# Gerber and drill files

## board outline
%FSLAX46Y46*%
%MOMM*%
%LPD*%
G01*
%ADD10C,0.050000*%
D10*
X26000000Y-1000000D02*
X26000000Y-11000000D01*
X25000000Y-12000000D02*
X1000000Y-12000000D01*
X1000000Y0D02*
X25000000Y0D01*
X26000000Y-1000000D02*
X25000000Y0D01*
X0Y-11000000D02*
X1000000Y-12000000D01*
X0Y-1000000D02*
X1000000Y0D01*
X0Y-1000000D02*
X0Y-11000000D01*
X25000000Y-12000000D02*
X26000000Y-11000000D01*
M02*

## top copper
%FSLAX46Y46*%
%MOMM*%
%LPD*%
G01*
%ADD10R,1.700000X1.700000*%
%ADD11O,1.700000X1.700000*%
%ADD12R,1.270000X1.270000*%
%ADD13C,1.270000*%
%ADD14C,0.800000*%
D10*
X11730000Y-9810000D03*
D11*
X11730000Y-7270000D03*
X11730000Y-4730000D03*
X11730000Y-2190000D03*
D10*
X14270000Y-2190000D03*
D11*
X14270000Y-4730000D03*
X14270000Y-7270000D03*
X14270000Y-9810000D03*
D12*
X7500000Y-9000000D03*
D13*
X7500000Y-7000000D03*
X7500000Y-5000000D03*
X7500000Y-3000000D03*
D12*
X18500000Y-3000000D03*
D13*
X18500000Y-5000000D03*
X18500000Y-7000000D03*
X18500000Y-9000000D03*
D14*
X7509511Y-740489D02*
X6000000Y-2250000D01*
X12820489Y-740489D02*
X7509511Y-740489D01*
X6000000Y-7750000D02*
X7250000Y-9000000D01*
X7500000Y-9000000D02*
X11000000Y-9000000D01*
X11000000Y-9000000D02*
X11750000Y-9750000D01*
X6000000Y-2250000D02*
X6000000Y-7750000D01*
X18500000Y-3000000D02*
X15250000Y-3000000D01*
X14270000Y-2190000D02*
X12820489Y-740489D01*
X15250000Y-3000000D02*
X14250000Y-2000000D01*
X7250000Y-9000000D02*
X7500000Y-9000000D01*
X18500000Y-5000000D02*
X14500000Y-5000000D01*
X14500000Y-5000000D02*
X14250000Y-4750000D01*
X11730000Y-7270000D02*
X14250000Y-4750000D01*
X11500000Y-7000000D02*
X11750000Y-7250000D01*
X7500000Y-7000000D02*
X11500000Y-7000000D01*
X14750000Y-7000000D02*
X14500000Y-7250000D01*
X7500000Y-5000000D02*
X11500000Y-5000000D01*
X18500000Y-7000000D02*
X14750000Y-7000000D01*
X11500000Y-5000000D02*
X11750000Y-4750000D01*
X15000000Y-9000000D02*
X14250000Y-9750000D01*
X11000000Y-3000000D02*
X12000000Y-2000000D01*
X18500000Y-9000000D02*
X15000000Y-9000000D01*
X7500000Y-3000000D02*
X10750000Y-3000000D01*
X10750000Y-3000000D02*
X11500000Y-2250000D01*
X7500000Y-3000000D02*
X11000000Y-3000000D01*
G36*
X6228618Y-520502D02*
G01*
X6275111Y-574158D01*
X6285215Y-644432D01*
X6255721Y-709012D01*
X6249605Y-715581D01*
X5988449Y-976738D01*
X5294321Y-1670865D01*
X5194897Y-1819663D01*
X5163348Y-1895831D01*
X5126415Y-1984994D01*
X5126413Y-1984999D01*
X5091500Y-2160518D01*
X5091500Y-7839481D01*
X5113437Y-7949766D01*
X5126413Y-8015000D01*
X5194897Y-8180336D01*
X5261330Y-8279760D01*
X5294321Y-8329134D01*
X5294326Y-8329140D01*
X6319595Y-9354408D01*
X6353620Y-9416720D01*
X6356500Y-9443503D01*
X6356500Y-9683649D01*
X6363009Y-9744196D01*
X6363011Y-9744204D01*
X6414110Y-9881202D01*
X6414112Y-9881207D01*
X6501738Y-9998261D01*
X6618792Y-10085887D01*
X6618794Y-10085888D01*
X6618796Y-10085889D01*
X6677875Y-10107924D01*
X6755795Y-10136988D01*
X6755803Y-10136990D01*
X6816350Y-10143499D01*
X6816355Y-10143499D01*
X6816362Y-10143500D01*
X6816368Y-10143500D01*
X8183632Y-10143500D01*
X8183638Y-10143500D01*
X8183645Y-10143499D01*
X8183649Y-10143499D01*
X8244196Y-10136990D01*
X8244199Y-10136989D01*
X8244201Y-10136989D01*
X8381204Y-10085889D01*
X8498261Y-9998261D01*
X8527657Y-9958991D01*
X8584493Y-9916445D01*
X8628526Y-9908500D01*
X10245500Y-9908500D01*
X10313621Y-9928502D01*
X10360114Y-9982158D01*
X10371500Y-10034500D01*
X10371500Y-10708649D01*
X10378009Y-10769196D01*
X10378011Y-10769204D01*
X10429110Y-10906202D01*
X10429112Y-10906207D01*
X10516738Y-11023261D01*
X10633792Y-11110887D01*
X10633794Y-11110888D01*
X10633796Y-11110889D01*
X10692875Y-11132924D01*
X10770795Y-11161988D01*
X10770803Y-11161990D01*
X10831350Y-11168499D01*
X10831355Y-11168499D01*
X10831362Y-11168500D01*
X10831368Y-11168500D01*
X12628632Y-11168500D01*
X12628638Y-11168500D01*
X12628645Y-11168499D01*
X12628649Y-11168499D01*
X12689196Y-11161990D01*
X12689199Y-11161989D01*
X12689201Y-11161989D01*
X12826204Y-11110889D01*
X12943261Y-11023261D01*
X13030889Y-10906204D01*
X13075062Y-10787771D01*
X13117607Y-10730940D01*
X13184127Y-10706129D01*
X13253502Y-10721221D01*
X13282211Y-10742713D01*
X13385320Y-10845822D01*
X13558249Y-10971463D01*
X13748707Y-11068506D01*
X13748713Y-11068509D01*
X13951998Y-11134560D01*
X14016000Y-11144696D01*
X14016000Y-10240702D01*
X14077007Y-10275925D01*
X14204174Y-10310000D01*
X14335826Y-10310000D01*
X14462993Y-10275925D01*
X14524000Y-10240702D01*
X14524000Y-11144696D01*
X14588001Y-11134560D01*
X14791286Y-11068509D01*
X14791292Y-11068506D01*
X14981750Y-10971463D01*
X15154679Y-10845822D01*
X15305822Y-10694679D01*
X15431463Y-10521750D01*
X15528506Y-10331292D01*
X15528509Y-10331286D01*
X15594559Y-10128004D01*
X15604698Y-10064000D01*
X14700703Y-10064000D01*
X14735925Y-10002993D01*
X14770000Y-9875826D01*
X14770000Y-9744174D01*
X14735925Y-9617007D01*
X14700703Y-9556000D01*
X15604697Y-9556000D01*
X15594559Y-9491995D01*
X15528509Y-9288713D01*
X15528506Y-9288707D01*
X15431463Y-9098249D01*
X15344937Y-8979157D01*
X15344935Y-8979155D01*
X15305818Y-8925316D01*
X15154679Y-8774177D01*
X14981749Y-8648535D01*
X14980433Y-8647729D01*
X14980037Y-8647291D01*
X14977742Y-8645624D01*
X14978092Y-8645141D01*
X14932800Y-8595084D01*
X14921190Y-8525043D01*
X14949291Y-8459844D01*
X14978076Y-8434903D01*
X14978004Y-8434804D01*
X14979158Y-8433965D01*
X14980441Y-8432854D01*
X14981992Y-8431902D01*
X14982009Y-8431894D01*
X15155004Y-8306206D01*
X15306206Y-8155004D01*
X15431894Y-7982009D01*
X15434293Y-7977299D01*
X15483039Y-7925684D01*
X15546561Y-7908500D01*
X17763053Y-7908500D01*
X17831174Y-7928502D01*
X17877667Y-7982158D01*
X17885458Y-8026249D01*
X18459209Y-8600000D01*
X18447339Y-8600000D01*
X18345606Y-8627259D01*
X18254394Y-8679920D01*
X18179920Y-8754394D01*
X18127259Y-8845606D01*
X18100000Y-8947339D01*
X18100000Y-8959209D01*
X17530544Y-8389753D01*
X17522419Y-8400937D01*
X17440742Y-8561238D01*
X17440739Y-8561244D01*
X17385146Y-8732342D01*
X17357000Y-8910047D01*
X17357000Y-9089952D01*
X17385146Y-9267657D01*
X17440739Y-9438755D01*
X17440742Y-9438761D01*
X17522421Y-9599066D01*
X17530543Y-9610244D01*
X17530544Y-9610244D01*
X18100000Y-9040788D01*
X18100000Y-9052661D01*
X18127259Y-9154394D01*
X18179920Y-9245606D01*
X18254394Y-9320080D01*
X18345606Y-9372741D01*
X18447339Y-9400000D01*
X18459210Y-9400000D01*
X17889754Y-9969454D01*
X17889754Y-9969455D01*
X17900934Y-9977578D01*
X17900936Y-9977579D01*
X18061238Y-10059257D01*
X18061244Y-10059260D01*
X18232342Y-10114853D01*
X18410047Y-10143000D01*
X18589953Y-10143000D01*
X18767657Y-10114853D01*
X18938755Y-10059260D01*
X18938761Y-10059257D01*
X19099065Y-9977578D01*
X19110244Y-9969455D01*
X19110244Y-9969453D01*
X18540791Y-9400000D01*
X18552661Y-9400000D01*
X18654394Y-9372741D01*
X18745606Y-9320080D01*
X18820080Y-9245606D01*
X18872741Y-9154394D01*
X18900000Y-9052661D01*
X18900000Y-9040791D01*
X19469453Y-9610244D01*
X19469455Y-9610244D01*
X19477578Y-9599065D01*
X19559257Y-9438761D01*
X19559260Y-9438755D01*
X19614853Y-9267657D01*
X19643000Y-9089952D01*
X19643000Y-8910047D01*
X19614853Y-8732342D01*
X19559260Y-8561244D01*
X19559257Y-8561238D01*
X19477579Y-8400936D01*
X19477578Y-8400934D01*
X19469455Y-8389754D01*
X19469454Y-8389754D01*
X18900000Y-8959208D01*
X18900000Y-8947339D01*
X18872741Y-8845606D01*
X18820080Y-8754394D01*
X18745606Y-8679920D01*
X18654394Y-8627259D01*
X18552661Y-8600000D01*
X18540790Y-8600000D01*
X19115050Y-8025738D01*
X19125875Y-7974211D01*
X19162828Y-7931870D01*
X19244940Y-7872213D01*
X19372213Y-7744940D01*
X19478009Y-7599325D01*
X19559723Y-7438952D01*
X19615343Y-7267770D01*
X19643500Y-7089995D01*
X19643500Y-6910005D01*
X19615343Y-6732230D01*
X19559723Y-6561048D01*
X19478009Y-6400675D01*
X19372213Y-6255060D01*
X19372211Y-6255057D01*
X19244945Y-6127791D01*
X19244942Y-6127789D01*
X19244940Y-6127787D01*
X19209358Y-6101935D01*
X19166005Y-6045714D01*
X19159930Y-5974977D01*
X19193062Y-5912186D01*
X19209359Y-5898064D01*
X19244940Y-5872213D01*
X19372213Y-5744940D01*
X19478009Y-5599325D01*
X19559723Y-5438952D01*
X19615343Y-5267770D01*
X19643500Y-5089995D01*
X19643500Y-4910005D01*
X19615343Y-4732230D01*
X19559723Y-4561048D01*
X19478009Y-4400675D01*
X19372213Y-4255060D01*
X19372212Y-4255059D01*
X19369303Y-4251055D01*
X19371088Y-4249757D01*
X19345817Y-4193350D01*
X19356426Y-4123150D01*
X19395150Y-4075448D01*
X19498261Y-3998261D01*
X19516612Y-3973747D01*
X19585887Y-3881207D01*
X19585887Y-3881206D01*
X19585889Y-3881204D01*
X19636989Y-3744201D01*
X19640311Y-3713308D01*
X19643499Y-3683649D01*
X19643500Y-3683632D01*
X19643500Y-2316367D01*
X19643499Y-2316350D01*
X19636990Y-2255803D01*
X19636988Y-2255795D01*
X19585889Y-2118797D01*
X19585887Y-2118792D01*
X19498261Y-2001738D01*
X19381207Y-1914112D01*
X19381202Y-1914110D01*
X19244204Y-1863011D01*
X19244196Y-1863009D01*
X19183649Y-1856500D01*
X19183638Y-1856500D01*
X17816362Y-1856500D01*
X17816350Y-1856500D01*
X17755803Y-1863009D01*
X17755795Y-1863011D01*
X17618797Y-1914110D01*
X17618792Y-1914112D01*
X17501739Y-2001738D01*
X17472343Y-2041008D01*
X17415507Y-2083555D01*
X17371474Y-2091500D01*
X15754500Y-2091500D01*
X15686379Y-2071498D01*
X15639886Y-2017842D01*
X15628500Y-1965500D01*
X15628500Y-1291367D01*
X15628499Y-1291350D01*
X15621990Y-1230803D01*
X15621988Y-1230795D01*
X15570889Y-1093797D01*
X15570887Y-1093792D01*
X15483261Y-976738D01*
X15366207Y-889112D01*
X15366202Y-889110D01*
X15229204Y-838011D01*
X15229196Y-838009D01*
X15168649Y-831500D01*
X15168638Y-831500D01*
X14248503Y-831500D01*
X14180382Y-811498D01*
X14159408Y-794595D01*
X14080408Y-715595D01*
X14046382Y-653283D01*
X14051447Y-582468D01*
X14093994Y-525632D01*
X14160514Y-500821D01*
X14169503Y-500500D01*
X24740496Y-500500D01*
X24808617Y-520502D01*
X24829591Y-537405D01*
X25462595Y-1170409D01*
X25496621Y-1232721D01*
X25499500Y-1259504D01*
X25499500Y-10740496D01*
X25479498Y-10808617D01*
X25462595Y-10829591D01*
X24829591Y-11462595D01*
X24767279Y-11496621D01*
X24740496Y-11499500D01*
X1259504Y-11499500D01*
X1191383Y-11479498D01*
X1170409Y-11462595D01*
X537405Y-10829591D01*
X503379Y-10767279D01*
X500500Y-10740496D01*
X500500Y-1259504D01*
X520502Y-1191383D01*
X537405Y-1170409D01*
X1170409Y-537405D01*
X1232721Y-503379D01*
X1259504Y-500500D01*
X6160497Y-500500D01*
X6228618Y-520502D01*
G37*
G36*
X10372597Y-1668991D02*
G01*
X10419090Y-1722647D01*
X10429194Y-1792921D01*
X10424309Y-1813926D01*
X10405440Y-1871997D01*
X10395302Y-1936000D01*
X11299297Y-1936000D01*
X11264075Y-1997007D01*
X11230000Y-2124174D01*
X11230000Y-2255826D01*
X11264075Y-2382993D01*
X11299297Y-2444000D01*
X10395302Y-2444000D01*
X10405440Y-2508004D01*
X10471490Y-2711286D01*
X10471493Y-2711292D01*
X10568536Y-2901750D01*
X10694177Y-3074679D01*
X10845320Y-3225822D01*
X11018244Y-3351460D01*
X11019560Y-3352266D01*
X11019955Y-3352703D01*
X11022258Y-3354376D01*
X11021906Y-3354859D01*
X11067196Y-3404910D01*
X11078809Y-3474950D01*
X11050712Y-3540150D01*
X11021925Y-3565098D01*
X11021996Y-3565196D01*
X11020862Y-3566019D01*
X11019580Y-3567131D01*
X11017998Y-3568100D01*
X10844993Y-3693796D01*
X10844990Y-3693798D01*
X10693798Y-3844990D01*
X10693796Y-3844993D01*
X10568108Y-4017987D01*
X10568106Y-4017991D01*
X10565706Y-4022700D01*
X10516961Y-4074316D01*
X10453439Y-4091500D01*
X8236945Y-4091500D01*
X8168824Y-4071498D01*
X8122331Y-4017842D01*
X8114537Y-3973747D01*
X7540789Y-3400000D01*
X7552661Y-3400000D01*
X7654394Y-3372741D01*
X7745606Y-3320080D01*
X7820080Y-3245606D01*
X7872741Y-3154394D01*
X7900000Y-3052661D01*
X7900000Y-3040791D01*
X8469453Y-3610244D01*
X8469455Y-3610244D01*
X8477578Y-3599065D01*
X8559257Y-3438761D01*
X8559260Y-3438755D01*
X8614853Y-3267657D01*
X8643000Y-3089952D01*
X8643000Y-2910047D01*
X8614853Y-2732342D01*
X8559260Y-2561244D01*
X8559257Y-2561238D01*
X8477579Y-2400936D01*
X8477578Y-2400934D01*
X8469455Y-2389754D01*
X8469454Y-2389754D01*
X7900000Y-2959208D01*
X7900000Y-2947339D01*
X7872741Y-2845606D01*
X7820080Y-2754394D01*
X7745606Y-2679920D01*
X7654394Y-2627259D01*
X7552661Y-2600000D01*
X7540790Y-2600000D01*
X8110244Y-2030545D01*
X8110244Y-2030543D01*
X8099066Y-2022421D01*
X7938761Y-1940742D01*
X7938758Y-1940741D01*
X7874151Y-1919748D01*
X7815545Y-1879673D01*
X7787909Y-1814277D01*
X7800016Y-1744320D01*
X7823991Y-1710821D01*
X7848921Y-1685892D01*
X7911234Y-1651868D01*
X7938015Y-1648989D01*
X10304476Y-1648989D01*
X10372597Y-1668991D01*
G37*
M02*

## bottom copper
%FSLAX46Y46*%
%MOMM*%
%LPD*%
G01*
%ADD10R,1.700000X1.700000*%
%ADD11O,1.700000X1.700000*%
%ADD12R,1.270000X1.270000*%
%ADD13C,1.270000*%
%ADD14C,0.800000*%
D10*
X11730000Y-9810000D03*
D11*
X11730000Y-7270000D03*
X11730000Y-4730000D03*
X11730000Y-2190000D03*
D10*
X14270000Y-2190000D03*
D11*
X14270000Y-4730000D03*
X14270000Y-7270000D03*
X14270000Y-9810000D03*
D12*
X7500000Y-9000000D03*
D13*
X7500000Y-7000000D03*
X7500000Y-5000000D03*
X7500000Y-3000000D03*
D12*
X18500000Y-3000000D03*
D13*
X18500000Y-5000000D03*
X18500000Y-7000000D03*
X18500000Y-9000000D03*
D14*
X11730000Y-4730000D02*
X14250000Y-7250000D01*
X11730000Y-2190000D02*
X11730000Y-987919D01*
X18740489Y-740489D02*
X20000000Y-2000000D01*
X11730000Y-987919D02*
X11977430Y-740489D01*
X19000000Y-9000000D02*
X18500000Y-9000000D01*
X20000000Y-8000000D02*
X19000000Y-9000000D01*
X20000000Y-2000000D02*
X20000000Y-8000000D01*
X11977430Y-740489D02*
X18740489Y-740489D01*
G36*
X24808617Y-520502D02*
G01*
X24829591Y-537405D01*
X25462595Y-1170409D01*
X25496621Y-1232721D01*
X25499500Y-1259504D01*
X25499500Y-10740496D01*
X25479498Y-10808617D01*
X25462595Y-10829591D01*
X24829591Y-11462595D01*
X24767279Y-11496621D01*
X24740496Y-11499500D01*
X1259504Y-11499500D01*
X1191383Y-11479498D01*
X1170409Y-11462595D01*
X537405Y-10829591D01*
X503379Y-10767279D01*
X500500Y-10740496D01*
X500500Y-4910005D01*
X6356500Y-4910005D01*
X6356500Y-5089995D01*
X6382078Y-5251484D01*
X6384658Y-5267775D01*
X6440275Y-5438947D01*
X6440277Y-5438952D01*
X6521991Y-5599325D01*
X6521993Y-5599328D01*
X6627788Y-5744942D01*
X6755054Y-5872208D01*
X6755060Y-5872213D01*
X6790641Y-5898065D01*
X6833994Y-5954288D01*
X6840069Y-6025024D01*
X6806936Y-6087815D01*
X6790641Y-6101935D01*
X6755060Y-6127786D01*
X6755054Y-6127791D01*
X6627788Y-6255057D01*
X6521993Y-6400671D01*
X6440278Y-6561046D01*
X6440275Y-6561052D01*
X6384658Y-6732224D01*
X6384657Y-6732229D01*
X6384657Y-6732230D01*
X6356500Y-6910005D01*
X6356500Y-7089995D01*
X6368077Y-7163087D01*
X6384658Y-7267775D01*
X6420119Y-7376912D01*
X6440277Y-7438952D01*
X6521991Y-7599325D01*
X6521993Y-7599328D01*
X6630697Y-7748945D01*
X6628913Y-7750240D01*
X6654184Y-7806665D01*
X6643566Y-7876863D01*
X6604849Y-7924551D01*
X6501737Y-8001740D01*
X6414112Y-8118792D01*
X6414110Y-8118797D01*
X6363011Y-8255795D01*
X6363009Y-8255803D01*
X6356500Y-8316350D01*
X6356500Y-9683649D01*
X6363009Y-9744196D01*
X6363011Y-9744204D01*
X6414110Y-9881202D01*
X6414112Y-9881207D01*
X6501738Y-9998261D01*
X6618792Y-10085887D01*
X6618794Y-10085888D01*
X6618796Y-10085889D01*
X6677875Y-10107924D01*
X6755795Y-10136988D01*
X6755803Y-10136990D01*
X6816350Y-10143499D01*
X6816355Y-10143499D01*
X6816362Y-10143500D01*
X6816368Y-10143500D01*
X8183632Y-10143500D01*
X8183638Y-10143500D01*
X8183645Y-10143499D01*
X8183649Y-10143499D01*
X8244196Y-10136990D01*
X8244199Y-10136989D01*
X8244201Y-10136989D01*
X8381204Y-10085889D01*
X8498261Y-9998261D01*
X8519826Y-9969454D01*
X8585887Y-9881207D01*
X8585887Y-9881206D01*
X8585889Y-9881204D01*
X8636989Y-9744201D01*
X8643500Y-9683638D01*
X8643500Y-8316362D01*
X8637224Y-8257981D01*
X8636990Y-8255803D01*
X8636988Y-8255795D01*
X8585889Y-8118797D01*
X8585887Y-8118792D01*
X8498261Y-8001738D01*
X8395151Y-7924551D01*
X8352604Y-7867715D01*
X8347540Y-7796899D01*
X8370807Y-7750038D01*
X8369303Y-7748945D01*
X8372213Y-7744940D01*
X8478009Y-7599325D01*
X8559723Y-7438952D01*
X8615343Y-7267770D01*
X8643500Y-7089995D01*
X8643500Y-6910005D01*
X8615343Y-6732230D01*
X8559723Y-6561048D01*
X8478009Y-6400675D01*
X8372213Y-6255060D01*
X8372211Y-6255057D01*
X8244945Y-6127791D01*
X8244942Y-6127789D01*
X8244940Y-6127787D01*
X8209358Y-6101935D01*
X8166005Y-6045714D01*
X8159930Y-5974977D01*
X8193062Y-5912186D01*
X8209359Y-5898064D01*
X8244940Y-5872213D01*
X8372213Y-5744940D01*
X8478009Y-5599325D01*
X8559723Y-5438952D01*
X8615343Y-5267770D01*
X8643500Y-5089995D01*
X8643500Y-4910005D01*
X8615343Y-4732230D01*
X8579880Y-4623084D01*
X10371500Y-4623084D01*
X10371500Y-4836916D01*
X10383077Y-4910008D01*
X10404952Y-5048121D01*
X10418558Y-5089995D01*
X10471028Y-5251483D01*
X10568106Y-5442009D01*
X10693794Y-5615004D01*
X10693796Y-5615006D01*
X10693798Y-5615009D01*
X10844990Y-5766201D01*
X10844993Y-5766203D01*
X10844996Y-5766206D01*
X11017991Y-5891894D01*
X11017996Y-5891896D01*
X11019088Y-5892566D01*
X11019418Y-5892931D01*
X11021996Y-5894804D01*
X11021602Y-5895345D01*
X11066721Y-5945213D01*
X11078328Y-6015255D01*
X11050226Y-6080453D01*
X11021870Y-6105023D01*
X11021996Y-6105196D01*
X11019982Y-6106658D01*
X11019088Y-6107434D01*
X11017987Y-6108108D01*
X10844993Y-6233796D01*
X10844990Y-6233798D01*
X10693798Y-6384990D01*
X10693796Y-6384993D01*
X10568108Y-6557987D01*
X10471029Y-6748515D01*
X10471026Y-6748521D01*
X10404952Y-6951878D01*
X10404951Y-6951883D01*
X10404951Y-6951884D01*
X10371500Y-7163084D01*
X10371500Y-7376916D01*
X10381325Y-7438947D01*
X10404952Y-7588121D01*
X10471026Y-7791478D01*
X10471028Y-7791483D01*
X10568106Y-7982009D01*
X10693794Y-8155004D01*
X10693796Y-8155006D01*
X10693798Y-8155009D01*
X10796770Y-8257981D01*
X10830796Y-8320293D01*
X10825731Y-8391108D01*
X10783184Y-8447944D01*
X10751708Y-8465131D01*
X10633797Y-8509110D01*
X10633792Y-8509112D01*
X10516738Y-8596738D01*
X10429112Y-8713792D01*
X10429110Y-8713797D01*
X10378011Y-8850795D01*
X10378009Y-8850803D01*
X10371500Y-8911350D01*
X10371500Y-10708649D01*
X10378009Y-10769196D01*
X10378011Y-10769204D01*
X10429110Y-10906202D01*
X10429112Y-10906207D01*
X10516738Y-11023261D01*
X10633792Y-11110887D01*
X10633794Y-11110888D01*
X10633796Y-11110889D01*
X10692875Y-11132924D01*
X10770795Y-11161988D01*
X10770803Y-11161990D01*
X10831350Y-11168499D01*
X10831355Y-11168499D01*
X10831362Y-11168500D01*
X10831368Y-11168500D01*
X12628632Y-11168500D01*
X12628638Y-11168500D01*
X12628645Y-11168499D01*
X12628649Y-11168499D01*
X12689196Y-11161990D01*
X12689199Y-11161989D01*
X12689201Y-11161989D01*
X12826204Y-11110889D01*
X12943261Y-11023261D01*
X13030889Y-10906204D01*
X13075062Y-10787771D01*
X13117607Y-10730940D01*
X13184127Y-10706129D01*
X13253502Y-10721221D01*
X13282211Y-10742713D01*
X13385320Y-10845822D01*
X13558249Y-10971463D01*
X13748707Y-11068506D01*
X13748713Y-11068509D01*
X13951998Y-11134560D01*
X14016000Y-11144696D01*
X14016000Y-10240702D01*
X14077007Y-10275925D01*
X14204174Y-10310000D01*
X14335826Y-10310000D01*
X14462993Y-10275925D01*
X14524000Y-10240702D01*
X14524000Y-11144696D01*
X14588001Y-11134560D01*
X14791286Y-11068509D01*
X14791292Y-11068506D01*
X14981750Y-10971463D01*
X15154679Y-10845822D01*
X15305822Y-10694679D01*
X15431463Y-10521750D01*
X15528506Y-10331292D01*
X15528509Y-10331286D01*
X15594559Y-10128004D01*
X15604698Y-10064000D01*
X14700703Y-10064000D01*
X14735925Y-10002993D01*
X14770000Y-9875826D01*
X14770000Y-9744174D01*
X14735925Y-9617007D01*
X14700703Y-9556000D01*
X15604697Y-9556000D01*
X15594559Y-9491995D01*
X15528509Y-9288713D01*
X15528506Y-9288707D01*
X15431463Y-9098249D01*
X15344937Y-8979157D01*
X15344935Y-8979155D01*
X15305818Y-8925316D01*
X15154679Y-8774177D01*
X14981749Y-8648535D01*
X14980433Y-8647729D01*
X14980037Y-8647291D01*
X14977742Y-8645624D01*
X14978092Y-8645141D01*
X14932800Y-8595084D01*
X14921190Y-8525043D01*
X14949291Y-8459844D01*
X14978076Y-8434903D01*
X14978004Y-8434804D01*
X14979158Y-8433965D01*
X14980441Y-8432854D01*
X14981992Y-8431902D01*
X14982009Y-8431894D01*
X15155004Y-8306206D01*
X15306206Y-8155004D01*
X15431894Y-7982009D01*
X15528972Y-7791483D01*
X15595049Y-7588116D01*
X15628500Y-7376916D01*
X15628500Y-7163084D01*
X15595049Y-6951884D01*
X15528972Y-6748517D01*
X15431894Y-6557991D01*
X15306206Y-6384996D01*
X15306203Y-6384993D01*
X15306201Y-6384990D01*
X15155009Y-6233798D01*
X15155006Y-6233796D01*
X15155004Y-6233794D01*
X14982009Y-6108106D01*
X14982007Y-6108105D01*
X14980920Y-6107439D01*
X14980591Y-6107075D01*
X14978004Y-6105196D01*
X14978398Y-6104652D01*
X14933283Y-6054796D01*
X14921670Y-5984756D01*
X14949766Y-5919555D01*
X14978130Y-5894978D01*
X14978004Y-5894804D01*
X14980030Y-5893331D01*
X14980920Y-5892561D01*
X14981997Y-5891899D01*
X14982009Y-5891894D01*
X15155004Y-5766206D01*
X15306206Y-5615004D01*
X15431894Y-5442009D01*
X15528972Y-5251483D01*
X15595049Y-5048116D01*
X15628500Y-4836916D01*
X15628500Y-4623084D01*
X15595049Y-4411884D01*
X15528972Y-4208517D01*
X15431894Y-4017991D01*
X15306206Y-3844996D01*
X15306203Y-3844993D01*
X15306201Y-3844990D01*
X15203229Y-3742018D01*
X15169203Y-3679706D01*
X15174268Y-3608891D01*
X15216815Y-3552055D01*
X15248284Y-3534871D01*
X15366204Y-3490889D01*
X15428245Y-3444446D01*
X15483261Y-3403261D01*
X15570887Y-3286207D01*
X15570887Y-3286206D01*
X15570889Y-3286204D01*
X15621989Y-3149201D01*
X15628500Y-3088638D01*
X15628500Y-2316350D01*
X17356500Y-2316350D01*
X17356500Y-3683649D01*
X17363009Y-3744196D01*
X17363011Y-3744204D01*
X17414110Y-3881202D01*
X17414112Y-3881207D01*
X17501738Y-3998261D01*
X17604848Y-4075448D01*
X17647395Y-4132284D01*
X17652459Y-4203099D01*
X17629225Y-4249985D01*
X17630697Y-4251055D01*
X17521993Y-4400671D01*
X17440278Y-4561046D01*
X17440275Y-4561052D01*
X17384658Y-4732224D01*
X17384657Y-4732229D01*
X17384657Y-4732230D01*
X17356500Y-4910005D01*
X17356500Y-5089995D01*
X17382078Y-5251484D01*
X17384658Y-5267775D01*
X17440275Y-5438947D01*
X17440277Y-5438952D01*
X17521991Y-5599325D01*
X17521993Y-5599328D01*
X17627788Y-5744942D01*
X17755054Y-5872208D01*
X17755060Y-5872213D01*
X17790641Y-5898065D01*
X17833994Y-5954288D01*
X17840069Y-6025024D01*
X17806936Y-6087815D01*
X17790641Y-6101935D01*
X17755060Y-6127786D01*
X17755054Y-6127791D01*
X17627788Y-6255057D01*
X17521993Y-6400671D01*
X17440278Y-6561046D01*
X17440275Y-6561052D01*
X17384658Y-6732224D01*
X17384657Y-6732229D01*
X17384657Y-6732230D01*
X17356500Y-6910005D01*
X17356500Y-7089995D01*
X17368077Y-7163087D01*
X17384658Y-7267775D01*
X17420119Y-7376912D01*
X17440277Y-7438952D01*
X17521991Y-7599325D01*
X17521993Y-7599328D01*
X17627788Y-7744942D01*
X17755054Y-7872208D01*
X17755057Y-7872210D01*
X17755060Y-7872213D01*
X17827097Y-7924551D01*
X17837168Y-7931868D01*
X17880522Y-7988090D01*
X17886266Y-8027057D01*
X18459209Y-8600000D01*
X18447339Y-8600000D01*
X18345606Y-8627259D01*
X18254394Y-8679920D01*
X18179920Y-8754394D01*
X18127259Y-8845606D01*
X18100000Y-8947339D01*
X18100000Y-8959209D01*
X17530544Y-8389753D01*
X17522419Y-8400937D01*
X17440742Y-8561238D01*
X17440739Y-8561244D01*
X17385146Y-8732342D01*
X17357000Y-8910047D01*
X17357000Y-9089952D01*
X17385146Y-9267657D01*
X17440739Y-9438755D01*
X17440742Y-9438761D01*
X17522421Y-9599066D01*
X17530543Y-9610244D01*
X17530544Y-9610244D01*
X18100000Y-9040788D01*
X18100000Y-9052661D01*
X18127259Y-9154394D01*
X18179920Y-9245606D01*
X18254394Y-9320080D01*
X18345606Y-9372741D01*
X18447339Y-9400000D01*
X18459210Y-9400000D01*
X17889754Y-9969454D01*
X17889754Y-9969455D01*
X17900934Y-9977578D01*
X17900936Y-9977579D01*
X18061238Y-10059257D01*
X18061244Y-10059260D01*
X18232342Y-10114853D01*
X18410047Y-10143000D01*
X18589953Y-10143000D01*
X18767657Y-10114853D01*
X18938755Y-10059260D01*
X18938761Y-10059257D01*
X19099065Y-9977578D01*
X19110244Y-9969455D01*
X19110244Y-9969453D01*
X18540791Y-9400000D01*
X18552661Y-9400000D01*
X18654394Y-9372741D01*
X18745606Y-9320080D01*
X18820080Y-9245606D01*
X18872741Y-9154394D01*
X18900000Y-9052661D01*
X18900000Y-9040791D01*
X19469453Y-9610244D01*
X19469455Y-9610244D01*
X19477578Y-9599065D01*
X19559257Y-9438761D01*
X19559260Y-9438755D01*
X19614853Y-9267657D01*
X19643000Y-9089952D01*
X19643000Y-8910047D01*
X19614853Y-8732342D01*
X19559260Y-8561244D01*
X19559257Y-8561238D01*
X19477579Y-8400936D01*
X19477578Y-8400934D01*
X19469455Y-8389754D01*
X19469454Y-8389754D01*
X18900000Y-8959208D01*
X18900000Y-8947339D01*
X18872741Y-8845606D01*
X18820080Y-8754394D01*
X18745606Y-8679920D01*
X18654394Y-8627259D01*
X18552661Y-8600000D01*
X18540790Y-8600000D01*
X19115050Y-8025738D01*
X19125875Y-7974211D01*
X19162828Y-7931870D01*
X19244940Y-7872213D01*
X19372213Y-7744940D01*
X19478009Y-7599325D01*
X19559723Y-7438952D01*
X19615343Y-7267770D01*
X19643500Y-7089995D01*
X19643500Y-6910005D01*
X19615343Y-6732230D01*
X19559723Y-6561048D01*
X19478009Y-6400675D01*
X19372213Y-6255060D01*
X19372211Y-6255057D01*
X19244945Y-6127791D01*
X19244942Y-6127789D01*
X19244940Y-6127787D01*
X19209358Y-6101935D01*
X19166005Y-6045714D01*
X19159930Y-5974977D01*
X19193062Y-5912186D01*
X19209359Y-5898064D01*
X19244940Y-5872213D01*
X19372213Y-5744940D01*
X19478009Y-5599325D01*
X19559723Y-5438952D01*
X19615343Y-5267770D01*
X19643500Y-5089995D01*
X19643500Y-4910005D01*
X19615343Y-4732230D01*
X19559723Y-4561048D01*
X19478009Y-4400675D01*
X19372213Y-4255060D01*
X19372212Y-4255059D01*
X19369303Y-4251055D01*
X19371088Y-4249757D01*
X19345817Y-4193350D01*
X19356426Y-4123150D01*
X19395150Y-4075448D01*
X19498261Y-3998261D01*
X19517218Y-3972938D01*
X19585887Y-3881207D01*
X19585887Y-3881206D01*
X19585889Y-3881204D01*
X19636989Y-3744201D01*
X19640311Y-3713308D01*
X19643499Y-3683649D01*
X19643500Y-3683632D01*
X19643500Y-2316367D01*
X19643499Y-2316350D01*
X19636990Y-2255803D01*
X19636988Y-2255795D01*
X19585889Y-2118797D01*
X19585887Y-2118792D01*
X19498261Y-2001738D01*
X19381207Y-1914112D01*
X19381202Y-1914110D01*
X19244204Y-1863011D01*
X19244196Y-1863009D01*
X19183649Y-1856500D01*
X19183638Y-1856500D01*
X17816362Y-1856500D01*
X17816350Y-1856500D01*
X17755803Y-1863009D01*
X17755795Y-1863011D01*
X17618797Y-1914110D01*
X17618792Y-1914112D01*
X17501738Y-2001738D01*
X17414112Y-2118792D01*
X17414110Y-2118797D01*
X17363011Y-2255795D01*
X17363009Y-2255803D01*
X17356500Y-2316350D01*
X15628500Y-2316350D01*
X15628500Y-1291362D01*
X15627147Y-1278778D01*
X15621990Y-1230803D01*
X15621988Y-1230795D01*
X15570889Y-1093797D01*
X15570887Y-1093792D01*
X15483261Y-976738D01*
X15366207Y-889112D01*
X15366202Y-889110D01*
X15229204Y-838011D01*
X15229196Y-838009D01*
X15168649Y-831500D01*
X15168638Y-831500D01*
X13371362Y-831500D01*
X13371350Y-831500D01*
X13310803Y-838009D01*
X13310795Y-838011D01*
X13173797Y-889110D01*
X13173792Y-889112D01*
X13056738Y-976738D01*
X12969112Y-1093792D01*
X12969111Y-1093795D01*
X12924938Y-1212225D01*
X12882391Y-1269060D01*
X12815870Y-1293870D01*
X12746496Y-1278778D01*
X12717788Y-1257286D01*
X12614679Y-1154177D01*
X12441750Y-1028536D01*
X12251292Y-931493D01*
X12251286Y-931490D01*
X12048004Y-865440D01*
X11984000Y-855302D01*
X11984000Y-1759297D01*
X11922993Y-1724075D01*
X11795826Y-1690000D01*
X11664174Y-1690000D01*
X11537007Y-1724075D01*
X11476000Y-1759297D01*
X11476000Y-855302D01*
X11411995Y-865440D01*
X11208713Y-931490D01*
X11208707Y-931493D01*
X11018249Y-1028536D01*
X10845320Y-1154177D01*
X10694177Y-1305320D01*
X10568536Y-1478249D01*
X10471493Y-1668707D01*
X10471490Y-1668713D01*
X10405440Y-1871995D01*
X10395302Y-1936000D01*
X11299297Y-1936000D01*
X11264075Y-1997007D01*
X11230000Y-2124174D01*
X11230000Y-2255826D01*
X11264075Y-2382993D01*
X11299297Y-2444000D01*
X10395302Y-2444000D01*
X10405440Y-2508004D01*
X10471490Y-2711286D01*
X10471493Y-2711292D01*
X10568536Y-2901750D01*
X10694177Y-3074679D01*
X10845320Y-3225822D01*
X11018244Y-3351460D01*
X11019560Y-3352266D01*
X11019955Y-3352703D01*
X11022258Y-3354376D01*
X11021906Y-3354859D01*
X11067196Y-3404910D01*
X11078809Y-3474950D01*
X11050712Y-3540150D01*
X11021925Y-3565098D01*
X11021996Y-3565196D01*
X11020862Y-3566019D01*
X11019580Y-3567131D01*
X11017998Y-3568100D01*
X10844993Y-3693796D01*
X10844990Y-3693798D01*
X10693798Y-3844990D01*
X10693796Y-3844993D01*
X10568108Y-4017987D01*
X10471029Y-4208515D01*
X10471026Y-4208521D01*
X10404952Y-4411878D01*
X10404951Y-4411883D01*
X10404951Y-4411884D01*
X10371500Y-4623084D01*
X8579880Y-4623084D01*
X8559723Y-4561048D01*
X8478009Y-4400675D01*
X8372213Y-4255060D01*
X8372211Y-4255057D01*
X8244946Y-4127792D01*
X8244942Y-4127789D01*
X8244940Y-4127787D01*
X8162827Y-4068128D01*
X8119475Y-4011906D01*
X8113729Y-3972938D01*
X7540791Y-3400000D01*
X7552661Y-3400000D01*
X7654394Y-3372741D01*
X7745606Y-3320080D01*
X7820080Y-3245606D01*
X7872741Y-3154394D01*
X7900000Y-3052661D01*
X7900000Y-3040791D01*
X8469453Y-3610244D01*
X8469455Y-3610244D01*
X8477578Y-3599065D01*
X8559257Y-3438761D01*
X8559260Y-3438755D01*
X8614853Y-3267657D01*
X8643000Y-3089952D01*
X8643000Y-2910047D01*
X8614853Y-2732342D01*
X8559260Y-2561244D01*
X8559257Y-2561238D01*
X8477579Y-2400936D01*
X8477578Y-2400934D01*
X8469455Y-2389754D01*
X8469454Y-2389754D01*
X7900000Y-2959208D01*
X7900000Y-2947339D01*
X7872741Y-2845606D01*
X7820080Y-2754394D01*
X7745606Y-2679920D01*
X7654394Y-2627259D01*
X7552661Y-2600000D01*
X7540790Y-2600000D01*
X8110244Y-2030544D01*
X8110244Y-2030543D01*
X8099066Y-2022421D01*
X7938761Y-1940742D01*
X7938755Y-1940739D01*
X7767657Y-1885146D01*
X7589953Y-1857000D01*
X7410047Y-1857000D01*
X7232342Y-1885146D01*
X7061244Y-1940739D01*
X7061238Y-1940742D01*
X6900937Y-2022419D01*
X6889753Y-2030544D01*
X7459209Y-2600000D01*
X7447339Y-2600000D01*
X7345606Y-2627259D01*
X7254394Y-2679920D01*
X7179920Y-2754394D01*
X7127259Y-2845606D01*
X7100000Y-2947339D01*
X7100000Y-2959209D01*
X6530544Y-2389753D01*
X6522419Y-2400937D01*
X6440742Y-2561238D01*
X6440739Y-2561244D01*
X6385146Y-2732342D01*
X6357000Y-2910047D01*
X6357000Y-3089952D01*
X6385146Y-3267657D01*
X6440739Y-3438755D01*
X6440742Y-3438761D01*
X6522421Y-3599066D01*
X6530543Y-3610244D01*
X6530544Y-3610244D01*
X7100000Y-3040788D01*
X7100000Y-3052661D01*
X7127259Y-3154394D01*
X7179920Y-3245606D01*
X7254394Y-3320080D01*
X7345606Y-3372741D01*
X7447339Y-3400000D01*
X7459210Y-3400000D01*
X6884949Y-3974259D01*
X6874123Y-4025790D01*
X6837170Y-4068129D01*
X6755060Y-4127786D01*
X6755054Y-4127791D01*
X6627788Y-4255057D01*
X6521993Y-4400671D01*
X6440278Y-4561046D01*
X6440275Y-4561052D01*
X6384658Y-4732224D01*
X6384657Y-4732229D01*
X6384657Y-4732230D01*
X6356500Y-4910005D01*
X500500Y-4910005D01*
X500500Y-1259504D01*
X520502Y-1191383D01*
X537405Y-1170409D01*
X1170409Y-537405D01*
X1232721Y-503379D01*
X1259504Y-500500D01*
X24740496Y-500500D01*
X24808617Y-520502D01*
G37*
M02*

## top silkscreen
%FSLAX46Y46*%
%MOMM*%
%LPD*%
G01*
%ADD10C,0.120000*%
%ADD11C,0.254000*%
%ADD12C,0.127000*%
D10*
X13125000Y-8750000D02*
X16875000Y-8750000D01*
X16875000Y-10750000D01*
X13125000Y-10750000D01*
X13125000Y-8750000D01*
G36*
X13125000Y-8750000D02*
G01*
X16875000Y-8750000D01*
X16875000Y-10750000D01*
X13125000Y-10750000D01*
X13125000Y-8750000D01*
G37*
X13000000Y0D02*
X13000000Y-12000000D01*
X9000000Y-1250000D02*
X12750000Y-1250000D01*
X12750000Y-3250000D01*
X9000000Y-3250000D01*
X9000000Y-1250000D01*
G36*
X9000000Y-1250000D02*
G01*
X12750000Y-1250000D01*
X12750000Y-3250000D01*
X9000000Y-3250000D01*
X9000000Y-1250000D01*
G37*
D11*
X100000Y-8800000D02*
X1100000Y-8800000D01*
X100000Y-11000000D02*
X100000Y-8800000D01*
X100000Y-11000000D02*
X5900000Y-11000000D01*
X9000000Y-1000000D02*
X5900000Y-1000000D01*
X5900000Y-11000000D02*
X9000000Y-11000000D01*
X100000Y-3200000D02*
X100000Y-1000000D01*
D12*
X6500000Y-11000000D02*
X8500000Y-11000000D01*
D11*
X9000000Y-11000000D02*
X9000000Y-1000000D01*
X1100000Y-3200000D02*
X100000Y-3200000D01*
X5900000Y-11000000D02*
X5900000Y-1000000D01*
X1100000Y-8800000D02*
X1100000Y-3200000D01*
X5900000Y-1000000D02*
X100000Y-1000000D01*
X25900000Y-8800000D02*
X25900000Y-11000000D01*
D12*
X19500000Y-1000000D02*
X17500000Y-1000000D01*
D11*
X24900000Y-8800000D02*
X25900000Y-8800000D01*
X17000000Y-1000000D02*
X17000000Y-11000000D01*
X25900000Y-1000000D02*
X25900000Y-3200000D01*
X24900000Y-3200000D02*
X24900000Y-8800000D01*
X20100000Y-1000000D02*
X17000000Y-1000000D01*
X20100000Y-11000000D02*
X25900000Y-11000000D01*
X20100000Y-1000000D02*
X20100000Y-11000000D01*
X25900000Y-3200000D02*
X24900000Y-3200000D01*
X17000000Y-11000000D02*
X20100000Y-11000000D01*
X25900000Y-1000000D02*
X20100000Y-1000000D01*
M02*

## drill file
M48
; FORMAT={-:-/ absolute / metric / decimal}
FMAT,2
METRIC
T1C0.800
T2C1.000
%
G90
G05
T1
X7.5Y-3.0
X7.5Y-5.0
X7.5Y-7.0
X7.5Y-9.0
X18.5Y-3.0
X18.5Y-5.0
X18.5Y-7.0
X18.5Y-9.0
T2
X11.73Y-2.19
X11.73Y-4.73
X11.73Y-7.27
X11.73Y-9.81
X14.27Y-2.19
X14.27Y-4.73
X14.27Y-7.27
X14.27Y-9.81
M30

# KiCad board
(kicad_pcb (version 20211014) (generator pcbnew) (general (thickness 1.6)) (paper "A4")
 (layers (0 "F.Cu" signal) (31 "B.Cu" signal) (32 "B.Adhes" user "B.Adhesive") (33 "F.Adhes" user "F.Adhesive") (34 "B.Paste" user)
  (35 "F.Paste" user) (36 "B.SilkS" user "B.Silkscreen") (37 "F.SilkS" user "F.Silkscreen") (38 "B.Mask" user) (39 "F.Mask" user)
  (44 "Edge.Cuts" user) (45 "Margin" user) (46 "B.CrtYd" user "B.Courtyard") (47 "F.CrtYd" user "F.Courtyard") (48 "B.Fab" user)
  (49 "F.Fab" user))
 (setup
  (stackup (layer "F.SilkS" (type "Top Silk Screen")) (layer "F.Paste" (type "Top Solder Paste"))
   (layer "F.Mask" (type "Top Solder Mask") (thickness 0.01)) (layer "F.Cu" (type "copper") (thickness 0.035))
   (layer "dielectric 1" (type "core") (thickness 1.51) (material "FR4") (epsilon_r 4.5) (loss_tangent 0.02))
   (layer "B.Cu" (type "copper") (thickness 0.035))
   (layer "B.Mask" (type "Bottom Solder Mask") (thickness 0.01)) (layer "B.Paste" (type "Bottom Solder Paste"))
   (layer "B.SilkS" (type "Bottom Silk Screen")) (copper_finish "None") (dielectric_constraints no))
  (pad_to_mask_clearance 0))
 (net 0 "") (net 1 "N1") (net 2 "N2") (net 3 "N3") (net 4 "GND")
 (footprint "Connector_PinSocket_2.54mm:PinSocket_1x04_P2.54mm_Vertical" (layer "F.Cu") (at 11.73 9.81 180)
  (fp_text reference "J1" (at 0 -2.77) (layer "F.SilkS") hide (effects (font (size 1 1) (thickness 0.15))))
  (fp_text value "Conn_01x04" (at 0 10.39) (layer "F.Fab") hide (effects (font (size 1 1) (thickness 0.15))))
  (pad "1" thru_hole rect (at 0 0 180) (size 1.7 1.7) (drill 1) (layers *.Cu *.Mask) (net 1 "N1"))
  (pad "2" thru_hole oval (at 0 2.54 180) (size 1.7 1.7) (drill 1) (layers *.Cu *.Mask) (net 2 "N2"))
  (pad "3" thru_hole oval (at 0 5.08 180) (size 1.7 1.7) (drill 1) (layers *.Cu *.Mask) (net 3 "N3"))
  (pad "4" thru_hole oval (at 0 7.62 180) (size 1.7 1.7) (drill 1) (layers *.Cu *.Mask) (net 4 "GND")))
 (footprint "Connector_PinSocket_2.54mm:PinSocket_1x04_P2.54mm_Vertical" (layer "F.Cu") (at 14.27 2.19)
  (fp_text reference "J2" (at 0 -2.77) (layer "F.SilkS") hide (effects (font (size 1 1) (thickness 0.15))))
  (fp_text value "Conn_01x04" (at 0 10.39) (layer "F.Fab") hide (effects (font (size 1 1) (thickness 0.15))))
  (pad "1" thru_hole rect (at 0 0) (size 1.7 1.7) (drill 1) (layers *.Cu *.Mask) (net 1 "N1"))
  (pad "2" thru_hole oval (at 0 2.54) (size 1.7 1.7) (drill 1) (layers *.Cu *.Mask) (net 2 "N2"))
  (pad "3" thru_hole oval (at 0 5.08) (size 1.7 1.7) (drill 1) (layers *.Cu *.Mask) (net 3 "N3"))
  (pad "4" thru_hole oval (at 0 7.62) (size 1.7 1.7) (drill 1) (layers *.Cu *.Mask) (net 4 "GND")))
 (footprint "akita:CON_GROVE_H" (layer "F.Cu") (at 7.5 6 90)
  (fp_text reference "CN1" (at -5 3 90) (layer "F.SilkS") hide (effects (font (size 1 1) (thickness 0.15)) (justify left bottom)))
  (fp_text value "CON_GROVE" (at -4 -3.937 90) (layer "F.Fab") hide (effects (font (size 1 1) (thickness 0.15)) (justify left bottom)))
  (fp_line (start -2.8 -7.4) (end -2.8 -6.4) (layer "F.SilkS") (width 0.254))
  (fp_line (start -5 -7.4) (end -2.8 -7.4) (layer "F.SilkS") (width 0.254))
  (fp_line (start -5 -7.4) (end -5 -1.6) (layer "F.SilkS") (width 0.254))
  (fp_line (start 5 1.5) (end 5 -1.6) (layer "F.SilkS") (width 0.254))
  (fp_line (start -5 -1.6) (end -5 1.5) (layer "F.SilkS") (width 0.254))
  (fp_line (start 2.8 -7.4) (end 5 -7.4) (layer "F.SilkS") (width 0.254))
  (fp_line (start -5 -1) (end -5 1) (layer "F.SilkS") (width 0.127))
  (fp_line (start -5 1.5) (end 5 1.5) (layer "F.SilkS") (width 0.254))
  (fp_line (start 2.8 -6.4) (end 2.8 -7.4) (layer "F.SilkS") (width 0.254))
  (fp_line (start -5 -1.6) (end 5 -1.6) (layer "F.SilkS") (width 0.254))
  (fp_line (start -2.8 -6.4) (end 2.8 -6.4) (layer "F.SilkS") (width 0.254))
  (fp_line (start 5 -1.6) (end 5 -7.4) (layer "F.SilkS") (width 0.254))
  (pad "1" thru_hole rect (at -3 0 90) (size 1.27 1.27) (drill 0.8) (layers *.Cu *.Mask) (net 1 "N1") (solder_mask_margin 0.1016))
  (pad "2" thru_hole circle (at -1 0 90) (size 1.27 1.27) (drill 0.8) (layers *.Cu *.Mask) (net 2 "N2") (solder_mask_margin 0.1016))
  (pad "3" thru_hole circle (at 1 0 90) (size 1.27 1.27) (drill 0.8) (layers *.Cu *.Mask) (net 3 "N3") (solder_mask_margin 0.1016))
  (pad "4" thru_hole circle (at 3 0 90) (size 1.27 1.27) (drill 0.8) (layers *.Cu *.Mask) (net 4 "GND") (solder_mask_margin 0.1016)))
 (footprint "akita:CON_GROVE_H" (layer "F.Cu") (at 18.5 6 -90)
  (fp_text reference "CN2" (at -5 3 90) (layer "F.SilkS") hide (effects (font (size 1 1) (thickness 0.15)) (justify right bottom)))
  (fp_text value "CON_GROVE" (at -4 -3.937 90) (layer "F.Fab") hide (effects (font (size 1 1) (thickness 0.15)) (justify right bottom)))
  (fp_line (start 2.8 -7.4) (end 5 -7.4) (layer "F.SilkS") (width 0.254))
  (fp_line (start -5 -1) (end -5 1) (layer "F.SilkS") (width 0.127))
  (fp_line (start 2.8 -6.4) (end 2.8 -7.4) (layer "F.SilkS") (width 0.254))
  (fp_line (start -5 1.5) (end 5 1.5) (layer "F.SilkS") (width 0.254))
  (fp_line (start -5 -7.4) (end -2.8 -7.4) (layer "F.SilkS") (width 0.254))
  (fp_line (start -2.8 -6.4) (end 2.8 -6.4) (layer "F.SilkS") (width 0.254))
  (fp_line (start -5 -1.6) (end -5 1.5) (layer "F.SilkS") (width 0.254))
  (fp_line (start 5 -1.6) (end 5 -7.4) (layer "F.SilkS") (width 0.254))
  (fp_line (start -5 -1.6) (end 5 -1.6) (layer "F.SilkS") (width 0.254))
  (fp_line (start -2.8 -7.4) (end -2.8 -6.4) (layer "F.SilkS") (width 0.254))
  (fp_line (start 5 1.5) (end 5 -1.6) (layer "F.SilkS") (width 0.254))
  (fp_line (start -5 -7.4) (end -5 -1.6) (layer "F.SilkS") (width 0.254))
  (pad "1" thru_hole rect (at -3 0 270) (size 1.27 1.27) (drill 0.8) (layers *.Cu *.Mask) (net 1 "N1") (solder_mask_margin 0.1016))
  (pad "2" thru_hole circle (at -1 0 270) (size 1.27 1.27) (drill 0.8) (layers *.Cu *.Mask) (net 2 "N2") (solder_mask_margin 0.1016))
  (pad "3" thru_hole circle (at 1 0 270) (size 1.27 1.27) (drill 0.8) (layers *.Cu *.Mask) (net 3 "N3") (solder_mask_margin 0.1016))
  (pad "4" thru_hole circle (at 3 0 270) (size 1.27 1.27) (drill 0.8) (layers *.Cu *.Mask) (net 4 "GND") (solder_mask_margin 0.1016)))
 (gr_rect (start 16.875 10.75) (end 13.125 8.75) (layer "F.SilkS") (width 0.12) (fill solid))
 (gr_line (start 13 0) (end 13 12) (layer "F.SilkS") (width 0.12))
 (gr_rect (start 12.75 3.25) (end 9 1.25) (layer "F.SilkS") (width 0.12) (fill solid))
 (gr_line (start 26 1) (end 26 11) (layer "Edge.Cuts") (width 0.05))
 (gr_line (start 25 12) (end 1 12) (layer "Edge.Cuts") (width 0.05))
 (gr_line (start 1 0) (end 25 0) (layer "Edge.Cuts") (width 0.05))
 (gr_line (start 26 1) (end 25 0) (layer "Edge.Cuts") (width 0.05))
 (gr_line (start 0 11) (end 1 12) (layer "Edge.Cuts") (width 0.05))
 (gr_line (start 0 1) (end 1 0) (layer "Edge.Cuts") (width 0.05))
 (gr_line (start 0 1) (end 0 11) (layer "Edge.Cuts") (width 0.05))
 (gr_line (start 25 12) (end 26 11) (layer "Edge.Cuts") (width 0.05))
 (segment (start 7.509511 0.740489) (end 6 2.25) (width 0.8) (layer "F.Cu") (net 1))
 (segment (start 12.820489 0.740489) (end 7.509511 0.740489) (width 0.8) (layer "F.Cu") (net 1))
 (segment (start 6 7.75) (end 7.25 9) (width 0.8) (layer "F.Cu") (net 1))
 (segment (start 7.5 9) (end 11 9) (width 0.8) (layer "F.Cu") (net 1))
 (segment (start 11 9) (end 11.75 9.75) (width 0.8) (layer "F.Cu") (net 1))
 (segment (start 6 2.25) (end 6 7.75) (width 0.8) (layer "F.Cu") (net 1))
 (segment (start 18.5 3) (end 15.25 3) (width 0.8) (layer "F.Cu") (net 1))
 (segment (start 14.27 2.19) (end 12.820489 0.740489) (width 0.8) (layer "F.Cu") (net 1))
 (segment (start 15.25 3) (end 14.25 2) (width 0.8) (layer "F.Cu") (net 1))
 (segment (start 7.25 9) (end 7.5 9) (width 0.8) (layer "F.Cu") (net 1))
 (segment (start 18.5 5) (end 14.5 5) (width 0.8) (layer "F.Cu") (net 2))
 (segment (start 14.5 5) (end 14.25 4.75) (width 0.8) (layer "F.Cu") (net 2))
 (segment (start 11.73 7.27) (end 14.25 4.75) (width 0.8) (layer "F.Cu") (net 2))
 (segment (start 11.5 7) (end 11.75 7.25) (width 0.8) (layer "F.Cu") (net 2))
 (segment (start 7.5 7) (end 11.5 7) (width 0.8) (layer "F.Cu") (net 2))
 (segment (start 14.75 7) (end 14.5 7.25) (width 0.8) (layer "F.Cu") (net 3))
 (segment (start 7.5 5) (end 11.5 5) (width 0.8) (layer "F.Cu") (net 3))
 (segment (start 18.5 7) (end 14.75 7) (width 0.8) (layer "F.Cu") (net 3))
 (segment (start 11.5 5) (end 11.75 4.75) (width 0.8) (layer "F.Cu") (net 3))
 (segment (start 11.73 4.73) (end 14.25 7.25) (width 0.8) (layer "B.Cu") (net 3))
 (segment (start 15 9) (end 14.25 9.75) (width 0.8) (layer "F.Cu") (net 4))
 (segment (start 11 3) (end 12 2) (width 0.8) (layer "F.Cu") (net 4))
 (segment (start 18.5 9) (end 15 9) (width 0.8) (layer "F.Cu") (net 4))
 (segment (start 7.5 3) (end 10.75 3) (width 0.8) (layer "F.Cu") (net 4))
 (segment (start 10.75 3) (end 11.5 2.25) (width 0.8) (layer "F.Cu") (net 4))
 (segment (start 7.5 3) (end 11 3) (width 0.8) (layer "F.Cu") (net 4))
 (segment (start 11.73 2.19) (end 11.73 0.987919) (width 0.8) (layer "B.Cu") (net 4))
 (segment (start 18.740489 0.740489) (end 20 2) (width 0.8) (layer "B.Cu") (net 4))
 (segment (start 11.73 0.987919) (end 11.97743 0.740489) (width 0.8) (layer "B.Cu") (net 4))
 (segment (start 19 9) (end 18.5 9) (width 0.8) (layer "B.Cu") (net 4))
 (segment (start 20 8) (end 19 9) (width 0.8) (layer "B.Cu") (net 4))
 (segment (start 20 2) (end 20 8) (width 0.8) (layer "B.Cu") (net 4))
 (segment (start 11.97743 0.740489) (end 18.740489 0.740489) (width 0.8) (layer "B.Cu") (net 4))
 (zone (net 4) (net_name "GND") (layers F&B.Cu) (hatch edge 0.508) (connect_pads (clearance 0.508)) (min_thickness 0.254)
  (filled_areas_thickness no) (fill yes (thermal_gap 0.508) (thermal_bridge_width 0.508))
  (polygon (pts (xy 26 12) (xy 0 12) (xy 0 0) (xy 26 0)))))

